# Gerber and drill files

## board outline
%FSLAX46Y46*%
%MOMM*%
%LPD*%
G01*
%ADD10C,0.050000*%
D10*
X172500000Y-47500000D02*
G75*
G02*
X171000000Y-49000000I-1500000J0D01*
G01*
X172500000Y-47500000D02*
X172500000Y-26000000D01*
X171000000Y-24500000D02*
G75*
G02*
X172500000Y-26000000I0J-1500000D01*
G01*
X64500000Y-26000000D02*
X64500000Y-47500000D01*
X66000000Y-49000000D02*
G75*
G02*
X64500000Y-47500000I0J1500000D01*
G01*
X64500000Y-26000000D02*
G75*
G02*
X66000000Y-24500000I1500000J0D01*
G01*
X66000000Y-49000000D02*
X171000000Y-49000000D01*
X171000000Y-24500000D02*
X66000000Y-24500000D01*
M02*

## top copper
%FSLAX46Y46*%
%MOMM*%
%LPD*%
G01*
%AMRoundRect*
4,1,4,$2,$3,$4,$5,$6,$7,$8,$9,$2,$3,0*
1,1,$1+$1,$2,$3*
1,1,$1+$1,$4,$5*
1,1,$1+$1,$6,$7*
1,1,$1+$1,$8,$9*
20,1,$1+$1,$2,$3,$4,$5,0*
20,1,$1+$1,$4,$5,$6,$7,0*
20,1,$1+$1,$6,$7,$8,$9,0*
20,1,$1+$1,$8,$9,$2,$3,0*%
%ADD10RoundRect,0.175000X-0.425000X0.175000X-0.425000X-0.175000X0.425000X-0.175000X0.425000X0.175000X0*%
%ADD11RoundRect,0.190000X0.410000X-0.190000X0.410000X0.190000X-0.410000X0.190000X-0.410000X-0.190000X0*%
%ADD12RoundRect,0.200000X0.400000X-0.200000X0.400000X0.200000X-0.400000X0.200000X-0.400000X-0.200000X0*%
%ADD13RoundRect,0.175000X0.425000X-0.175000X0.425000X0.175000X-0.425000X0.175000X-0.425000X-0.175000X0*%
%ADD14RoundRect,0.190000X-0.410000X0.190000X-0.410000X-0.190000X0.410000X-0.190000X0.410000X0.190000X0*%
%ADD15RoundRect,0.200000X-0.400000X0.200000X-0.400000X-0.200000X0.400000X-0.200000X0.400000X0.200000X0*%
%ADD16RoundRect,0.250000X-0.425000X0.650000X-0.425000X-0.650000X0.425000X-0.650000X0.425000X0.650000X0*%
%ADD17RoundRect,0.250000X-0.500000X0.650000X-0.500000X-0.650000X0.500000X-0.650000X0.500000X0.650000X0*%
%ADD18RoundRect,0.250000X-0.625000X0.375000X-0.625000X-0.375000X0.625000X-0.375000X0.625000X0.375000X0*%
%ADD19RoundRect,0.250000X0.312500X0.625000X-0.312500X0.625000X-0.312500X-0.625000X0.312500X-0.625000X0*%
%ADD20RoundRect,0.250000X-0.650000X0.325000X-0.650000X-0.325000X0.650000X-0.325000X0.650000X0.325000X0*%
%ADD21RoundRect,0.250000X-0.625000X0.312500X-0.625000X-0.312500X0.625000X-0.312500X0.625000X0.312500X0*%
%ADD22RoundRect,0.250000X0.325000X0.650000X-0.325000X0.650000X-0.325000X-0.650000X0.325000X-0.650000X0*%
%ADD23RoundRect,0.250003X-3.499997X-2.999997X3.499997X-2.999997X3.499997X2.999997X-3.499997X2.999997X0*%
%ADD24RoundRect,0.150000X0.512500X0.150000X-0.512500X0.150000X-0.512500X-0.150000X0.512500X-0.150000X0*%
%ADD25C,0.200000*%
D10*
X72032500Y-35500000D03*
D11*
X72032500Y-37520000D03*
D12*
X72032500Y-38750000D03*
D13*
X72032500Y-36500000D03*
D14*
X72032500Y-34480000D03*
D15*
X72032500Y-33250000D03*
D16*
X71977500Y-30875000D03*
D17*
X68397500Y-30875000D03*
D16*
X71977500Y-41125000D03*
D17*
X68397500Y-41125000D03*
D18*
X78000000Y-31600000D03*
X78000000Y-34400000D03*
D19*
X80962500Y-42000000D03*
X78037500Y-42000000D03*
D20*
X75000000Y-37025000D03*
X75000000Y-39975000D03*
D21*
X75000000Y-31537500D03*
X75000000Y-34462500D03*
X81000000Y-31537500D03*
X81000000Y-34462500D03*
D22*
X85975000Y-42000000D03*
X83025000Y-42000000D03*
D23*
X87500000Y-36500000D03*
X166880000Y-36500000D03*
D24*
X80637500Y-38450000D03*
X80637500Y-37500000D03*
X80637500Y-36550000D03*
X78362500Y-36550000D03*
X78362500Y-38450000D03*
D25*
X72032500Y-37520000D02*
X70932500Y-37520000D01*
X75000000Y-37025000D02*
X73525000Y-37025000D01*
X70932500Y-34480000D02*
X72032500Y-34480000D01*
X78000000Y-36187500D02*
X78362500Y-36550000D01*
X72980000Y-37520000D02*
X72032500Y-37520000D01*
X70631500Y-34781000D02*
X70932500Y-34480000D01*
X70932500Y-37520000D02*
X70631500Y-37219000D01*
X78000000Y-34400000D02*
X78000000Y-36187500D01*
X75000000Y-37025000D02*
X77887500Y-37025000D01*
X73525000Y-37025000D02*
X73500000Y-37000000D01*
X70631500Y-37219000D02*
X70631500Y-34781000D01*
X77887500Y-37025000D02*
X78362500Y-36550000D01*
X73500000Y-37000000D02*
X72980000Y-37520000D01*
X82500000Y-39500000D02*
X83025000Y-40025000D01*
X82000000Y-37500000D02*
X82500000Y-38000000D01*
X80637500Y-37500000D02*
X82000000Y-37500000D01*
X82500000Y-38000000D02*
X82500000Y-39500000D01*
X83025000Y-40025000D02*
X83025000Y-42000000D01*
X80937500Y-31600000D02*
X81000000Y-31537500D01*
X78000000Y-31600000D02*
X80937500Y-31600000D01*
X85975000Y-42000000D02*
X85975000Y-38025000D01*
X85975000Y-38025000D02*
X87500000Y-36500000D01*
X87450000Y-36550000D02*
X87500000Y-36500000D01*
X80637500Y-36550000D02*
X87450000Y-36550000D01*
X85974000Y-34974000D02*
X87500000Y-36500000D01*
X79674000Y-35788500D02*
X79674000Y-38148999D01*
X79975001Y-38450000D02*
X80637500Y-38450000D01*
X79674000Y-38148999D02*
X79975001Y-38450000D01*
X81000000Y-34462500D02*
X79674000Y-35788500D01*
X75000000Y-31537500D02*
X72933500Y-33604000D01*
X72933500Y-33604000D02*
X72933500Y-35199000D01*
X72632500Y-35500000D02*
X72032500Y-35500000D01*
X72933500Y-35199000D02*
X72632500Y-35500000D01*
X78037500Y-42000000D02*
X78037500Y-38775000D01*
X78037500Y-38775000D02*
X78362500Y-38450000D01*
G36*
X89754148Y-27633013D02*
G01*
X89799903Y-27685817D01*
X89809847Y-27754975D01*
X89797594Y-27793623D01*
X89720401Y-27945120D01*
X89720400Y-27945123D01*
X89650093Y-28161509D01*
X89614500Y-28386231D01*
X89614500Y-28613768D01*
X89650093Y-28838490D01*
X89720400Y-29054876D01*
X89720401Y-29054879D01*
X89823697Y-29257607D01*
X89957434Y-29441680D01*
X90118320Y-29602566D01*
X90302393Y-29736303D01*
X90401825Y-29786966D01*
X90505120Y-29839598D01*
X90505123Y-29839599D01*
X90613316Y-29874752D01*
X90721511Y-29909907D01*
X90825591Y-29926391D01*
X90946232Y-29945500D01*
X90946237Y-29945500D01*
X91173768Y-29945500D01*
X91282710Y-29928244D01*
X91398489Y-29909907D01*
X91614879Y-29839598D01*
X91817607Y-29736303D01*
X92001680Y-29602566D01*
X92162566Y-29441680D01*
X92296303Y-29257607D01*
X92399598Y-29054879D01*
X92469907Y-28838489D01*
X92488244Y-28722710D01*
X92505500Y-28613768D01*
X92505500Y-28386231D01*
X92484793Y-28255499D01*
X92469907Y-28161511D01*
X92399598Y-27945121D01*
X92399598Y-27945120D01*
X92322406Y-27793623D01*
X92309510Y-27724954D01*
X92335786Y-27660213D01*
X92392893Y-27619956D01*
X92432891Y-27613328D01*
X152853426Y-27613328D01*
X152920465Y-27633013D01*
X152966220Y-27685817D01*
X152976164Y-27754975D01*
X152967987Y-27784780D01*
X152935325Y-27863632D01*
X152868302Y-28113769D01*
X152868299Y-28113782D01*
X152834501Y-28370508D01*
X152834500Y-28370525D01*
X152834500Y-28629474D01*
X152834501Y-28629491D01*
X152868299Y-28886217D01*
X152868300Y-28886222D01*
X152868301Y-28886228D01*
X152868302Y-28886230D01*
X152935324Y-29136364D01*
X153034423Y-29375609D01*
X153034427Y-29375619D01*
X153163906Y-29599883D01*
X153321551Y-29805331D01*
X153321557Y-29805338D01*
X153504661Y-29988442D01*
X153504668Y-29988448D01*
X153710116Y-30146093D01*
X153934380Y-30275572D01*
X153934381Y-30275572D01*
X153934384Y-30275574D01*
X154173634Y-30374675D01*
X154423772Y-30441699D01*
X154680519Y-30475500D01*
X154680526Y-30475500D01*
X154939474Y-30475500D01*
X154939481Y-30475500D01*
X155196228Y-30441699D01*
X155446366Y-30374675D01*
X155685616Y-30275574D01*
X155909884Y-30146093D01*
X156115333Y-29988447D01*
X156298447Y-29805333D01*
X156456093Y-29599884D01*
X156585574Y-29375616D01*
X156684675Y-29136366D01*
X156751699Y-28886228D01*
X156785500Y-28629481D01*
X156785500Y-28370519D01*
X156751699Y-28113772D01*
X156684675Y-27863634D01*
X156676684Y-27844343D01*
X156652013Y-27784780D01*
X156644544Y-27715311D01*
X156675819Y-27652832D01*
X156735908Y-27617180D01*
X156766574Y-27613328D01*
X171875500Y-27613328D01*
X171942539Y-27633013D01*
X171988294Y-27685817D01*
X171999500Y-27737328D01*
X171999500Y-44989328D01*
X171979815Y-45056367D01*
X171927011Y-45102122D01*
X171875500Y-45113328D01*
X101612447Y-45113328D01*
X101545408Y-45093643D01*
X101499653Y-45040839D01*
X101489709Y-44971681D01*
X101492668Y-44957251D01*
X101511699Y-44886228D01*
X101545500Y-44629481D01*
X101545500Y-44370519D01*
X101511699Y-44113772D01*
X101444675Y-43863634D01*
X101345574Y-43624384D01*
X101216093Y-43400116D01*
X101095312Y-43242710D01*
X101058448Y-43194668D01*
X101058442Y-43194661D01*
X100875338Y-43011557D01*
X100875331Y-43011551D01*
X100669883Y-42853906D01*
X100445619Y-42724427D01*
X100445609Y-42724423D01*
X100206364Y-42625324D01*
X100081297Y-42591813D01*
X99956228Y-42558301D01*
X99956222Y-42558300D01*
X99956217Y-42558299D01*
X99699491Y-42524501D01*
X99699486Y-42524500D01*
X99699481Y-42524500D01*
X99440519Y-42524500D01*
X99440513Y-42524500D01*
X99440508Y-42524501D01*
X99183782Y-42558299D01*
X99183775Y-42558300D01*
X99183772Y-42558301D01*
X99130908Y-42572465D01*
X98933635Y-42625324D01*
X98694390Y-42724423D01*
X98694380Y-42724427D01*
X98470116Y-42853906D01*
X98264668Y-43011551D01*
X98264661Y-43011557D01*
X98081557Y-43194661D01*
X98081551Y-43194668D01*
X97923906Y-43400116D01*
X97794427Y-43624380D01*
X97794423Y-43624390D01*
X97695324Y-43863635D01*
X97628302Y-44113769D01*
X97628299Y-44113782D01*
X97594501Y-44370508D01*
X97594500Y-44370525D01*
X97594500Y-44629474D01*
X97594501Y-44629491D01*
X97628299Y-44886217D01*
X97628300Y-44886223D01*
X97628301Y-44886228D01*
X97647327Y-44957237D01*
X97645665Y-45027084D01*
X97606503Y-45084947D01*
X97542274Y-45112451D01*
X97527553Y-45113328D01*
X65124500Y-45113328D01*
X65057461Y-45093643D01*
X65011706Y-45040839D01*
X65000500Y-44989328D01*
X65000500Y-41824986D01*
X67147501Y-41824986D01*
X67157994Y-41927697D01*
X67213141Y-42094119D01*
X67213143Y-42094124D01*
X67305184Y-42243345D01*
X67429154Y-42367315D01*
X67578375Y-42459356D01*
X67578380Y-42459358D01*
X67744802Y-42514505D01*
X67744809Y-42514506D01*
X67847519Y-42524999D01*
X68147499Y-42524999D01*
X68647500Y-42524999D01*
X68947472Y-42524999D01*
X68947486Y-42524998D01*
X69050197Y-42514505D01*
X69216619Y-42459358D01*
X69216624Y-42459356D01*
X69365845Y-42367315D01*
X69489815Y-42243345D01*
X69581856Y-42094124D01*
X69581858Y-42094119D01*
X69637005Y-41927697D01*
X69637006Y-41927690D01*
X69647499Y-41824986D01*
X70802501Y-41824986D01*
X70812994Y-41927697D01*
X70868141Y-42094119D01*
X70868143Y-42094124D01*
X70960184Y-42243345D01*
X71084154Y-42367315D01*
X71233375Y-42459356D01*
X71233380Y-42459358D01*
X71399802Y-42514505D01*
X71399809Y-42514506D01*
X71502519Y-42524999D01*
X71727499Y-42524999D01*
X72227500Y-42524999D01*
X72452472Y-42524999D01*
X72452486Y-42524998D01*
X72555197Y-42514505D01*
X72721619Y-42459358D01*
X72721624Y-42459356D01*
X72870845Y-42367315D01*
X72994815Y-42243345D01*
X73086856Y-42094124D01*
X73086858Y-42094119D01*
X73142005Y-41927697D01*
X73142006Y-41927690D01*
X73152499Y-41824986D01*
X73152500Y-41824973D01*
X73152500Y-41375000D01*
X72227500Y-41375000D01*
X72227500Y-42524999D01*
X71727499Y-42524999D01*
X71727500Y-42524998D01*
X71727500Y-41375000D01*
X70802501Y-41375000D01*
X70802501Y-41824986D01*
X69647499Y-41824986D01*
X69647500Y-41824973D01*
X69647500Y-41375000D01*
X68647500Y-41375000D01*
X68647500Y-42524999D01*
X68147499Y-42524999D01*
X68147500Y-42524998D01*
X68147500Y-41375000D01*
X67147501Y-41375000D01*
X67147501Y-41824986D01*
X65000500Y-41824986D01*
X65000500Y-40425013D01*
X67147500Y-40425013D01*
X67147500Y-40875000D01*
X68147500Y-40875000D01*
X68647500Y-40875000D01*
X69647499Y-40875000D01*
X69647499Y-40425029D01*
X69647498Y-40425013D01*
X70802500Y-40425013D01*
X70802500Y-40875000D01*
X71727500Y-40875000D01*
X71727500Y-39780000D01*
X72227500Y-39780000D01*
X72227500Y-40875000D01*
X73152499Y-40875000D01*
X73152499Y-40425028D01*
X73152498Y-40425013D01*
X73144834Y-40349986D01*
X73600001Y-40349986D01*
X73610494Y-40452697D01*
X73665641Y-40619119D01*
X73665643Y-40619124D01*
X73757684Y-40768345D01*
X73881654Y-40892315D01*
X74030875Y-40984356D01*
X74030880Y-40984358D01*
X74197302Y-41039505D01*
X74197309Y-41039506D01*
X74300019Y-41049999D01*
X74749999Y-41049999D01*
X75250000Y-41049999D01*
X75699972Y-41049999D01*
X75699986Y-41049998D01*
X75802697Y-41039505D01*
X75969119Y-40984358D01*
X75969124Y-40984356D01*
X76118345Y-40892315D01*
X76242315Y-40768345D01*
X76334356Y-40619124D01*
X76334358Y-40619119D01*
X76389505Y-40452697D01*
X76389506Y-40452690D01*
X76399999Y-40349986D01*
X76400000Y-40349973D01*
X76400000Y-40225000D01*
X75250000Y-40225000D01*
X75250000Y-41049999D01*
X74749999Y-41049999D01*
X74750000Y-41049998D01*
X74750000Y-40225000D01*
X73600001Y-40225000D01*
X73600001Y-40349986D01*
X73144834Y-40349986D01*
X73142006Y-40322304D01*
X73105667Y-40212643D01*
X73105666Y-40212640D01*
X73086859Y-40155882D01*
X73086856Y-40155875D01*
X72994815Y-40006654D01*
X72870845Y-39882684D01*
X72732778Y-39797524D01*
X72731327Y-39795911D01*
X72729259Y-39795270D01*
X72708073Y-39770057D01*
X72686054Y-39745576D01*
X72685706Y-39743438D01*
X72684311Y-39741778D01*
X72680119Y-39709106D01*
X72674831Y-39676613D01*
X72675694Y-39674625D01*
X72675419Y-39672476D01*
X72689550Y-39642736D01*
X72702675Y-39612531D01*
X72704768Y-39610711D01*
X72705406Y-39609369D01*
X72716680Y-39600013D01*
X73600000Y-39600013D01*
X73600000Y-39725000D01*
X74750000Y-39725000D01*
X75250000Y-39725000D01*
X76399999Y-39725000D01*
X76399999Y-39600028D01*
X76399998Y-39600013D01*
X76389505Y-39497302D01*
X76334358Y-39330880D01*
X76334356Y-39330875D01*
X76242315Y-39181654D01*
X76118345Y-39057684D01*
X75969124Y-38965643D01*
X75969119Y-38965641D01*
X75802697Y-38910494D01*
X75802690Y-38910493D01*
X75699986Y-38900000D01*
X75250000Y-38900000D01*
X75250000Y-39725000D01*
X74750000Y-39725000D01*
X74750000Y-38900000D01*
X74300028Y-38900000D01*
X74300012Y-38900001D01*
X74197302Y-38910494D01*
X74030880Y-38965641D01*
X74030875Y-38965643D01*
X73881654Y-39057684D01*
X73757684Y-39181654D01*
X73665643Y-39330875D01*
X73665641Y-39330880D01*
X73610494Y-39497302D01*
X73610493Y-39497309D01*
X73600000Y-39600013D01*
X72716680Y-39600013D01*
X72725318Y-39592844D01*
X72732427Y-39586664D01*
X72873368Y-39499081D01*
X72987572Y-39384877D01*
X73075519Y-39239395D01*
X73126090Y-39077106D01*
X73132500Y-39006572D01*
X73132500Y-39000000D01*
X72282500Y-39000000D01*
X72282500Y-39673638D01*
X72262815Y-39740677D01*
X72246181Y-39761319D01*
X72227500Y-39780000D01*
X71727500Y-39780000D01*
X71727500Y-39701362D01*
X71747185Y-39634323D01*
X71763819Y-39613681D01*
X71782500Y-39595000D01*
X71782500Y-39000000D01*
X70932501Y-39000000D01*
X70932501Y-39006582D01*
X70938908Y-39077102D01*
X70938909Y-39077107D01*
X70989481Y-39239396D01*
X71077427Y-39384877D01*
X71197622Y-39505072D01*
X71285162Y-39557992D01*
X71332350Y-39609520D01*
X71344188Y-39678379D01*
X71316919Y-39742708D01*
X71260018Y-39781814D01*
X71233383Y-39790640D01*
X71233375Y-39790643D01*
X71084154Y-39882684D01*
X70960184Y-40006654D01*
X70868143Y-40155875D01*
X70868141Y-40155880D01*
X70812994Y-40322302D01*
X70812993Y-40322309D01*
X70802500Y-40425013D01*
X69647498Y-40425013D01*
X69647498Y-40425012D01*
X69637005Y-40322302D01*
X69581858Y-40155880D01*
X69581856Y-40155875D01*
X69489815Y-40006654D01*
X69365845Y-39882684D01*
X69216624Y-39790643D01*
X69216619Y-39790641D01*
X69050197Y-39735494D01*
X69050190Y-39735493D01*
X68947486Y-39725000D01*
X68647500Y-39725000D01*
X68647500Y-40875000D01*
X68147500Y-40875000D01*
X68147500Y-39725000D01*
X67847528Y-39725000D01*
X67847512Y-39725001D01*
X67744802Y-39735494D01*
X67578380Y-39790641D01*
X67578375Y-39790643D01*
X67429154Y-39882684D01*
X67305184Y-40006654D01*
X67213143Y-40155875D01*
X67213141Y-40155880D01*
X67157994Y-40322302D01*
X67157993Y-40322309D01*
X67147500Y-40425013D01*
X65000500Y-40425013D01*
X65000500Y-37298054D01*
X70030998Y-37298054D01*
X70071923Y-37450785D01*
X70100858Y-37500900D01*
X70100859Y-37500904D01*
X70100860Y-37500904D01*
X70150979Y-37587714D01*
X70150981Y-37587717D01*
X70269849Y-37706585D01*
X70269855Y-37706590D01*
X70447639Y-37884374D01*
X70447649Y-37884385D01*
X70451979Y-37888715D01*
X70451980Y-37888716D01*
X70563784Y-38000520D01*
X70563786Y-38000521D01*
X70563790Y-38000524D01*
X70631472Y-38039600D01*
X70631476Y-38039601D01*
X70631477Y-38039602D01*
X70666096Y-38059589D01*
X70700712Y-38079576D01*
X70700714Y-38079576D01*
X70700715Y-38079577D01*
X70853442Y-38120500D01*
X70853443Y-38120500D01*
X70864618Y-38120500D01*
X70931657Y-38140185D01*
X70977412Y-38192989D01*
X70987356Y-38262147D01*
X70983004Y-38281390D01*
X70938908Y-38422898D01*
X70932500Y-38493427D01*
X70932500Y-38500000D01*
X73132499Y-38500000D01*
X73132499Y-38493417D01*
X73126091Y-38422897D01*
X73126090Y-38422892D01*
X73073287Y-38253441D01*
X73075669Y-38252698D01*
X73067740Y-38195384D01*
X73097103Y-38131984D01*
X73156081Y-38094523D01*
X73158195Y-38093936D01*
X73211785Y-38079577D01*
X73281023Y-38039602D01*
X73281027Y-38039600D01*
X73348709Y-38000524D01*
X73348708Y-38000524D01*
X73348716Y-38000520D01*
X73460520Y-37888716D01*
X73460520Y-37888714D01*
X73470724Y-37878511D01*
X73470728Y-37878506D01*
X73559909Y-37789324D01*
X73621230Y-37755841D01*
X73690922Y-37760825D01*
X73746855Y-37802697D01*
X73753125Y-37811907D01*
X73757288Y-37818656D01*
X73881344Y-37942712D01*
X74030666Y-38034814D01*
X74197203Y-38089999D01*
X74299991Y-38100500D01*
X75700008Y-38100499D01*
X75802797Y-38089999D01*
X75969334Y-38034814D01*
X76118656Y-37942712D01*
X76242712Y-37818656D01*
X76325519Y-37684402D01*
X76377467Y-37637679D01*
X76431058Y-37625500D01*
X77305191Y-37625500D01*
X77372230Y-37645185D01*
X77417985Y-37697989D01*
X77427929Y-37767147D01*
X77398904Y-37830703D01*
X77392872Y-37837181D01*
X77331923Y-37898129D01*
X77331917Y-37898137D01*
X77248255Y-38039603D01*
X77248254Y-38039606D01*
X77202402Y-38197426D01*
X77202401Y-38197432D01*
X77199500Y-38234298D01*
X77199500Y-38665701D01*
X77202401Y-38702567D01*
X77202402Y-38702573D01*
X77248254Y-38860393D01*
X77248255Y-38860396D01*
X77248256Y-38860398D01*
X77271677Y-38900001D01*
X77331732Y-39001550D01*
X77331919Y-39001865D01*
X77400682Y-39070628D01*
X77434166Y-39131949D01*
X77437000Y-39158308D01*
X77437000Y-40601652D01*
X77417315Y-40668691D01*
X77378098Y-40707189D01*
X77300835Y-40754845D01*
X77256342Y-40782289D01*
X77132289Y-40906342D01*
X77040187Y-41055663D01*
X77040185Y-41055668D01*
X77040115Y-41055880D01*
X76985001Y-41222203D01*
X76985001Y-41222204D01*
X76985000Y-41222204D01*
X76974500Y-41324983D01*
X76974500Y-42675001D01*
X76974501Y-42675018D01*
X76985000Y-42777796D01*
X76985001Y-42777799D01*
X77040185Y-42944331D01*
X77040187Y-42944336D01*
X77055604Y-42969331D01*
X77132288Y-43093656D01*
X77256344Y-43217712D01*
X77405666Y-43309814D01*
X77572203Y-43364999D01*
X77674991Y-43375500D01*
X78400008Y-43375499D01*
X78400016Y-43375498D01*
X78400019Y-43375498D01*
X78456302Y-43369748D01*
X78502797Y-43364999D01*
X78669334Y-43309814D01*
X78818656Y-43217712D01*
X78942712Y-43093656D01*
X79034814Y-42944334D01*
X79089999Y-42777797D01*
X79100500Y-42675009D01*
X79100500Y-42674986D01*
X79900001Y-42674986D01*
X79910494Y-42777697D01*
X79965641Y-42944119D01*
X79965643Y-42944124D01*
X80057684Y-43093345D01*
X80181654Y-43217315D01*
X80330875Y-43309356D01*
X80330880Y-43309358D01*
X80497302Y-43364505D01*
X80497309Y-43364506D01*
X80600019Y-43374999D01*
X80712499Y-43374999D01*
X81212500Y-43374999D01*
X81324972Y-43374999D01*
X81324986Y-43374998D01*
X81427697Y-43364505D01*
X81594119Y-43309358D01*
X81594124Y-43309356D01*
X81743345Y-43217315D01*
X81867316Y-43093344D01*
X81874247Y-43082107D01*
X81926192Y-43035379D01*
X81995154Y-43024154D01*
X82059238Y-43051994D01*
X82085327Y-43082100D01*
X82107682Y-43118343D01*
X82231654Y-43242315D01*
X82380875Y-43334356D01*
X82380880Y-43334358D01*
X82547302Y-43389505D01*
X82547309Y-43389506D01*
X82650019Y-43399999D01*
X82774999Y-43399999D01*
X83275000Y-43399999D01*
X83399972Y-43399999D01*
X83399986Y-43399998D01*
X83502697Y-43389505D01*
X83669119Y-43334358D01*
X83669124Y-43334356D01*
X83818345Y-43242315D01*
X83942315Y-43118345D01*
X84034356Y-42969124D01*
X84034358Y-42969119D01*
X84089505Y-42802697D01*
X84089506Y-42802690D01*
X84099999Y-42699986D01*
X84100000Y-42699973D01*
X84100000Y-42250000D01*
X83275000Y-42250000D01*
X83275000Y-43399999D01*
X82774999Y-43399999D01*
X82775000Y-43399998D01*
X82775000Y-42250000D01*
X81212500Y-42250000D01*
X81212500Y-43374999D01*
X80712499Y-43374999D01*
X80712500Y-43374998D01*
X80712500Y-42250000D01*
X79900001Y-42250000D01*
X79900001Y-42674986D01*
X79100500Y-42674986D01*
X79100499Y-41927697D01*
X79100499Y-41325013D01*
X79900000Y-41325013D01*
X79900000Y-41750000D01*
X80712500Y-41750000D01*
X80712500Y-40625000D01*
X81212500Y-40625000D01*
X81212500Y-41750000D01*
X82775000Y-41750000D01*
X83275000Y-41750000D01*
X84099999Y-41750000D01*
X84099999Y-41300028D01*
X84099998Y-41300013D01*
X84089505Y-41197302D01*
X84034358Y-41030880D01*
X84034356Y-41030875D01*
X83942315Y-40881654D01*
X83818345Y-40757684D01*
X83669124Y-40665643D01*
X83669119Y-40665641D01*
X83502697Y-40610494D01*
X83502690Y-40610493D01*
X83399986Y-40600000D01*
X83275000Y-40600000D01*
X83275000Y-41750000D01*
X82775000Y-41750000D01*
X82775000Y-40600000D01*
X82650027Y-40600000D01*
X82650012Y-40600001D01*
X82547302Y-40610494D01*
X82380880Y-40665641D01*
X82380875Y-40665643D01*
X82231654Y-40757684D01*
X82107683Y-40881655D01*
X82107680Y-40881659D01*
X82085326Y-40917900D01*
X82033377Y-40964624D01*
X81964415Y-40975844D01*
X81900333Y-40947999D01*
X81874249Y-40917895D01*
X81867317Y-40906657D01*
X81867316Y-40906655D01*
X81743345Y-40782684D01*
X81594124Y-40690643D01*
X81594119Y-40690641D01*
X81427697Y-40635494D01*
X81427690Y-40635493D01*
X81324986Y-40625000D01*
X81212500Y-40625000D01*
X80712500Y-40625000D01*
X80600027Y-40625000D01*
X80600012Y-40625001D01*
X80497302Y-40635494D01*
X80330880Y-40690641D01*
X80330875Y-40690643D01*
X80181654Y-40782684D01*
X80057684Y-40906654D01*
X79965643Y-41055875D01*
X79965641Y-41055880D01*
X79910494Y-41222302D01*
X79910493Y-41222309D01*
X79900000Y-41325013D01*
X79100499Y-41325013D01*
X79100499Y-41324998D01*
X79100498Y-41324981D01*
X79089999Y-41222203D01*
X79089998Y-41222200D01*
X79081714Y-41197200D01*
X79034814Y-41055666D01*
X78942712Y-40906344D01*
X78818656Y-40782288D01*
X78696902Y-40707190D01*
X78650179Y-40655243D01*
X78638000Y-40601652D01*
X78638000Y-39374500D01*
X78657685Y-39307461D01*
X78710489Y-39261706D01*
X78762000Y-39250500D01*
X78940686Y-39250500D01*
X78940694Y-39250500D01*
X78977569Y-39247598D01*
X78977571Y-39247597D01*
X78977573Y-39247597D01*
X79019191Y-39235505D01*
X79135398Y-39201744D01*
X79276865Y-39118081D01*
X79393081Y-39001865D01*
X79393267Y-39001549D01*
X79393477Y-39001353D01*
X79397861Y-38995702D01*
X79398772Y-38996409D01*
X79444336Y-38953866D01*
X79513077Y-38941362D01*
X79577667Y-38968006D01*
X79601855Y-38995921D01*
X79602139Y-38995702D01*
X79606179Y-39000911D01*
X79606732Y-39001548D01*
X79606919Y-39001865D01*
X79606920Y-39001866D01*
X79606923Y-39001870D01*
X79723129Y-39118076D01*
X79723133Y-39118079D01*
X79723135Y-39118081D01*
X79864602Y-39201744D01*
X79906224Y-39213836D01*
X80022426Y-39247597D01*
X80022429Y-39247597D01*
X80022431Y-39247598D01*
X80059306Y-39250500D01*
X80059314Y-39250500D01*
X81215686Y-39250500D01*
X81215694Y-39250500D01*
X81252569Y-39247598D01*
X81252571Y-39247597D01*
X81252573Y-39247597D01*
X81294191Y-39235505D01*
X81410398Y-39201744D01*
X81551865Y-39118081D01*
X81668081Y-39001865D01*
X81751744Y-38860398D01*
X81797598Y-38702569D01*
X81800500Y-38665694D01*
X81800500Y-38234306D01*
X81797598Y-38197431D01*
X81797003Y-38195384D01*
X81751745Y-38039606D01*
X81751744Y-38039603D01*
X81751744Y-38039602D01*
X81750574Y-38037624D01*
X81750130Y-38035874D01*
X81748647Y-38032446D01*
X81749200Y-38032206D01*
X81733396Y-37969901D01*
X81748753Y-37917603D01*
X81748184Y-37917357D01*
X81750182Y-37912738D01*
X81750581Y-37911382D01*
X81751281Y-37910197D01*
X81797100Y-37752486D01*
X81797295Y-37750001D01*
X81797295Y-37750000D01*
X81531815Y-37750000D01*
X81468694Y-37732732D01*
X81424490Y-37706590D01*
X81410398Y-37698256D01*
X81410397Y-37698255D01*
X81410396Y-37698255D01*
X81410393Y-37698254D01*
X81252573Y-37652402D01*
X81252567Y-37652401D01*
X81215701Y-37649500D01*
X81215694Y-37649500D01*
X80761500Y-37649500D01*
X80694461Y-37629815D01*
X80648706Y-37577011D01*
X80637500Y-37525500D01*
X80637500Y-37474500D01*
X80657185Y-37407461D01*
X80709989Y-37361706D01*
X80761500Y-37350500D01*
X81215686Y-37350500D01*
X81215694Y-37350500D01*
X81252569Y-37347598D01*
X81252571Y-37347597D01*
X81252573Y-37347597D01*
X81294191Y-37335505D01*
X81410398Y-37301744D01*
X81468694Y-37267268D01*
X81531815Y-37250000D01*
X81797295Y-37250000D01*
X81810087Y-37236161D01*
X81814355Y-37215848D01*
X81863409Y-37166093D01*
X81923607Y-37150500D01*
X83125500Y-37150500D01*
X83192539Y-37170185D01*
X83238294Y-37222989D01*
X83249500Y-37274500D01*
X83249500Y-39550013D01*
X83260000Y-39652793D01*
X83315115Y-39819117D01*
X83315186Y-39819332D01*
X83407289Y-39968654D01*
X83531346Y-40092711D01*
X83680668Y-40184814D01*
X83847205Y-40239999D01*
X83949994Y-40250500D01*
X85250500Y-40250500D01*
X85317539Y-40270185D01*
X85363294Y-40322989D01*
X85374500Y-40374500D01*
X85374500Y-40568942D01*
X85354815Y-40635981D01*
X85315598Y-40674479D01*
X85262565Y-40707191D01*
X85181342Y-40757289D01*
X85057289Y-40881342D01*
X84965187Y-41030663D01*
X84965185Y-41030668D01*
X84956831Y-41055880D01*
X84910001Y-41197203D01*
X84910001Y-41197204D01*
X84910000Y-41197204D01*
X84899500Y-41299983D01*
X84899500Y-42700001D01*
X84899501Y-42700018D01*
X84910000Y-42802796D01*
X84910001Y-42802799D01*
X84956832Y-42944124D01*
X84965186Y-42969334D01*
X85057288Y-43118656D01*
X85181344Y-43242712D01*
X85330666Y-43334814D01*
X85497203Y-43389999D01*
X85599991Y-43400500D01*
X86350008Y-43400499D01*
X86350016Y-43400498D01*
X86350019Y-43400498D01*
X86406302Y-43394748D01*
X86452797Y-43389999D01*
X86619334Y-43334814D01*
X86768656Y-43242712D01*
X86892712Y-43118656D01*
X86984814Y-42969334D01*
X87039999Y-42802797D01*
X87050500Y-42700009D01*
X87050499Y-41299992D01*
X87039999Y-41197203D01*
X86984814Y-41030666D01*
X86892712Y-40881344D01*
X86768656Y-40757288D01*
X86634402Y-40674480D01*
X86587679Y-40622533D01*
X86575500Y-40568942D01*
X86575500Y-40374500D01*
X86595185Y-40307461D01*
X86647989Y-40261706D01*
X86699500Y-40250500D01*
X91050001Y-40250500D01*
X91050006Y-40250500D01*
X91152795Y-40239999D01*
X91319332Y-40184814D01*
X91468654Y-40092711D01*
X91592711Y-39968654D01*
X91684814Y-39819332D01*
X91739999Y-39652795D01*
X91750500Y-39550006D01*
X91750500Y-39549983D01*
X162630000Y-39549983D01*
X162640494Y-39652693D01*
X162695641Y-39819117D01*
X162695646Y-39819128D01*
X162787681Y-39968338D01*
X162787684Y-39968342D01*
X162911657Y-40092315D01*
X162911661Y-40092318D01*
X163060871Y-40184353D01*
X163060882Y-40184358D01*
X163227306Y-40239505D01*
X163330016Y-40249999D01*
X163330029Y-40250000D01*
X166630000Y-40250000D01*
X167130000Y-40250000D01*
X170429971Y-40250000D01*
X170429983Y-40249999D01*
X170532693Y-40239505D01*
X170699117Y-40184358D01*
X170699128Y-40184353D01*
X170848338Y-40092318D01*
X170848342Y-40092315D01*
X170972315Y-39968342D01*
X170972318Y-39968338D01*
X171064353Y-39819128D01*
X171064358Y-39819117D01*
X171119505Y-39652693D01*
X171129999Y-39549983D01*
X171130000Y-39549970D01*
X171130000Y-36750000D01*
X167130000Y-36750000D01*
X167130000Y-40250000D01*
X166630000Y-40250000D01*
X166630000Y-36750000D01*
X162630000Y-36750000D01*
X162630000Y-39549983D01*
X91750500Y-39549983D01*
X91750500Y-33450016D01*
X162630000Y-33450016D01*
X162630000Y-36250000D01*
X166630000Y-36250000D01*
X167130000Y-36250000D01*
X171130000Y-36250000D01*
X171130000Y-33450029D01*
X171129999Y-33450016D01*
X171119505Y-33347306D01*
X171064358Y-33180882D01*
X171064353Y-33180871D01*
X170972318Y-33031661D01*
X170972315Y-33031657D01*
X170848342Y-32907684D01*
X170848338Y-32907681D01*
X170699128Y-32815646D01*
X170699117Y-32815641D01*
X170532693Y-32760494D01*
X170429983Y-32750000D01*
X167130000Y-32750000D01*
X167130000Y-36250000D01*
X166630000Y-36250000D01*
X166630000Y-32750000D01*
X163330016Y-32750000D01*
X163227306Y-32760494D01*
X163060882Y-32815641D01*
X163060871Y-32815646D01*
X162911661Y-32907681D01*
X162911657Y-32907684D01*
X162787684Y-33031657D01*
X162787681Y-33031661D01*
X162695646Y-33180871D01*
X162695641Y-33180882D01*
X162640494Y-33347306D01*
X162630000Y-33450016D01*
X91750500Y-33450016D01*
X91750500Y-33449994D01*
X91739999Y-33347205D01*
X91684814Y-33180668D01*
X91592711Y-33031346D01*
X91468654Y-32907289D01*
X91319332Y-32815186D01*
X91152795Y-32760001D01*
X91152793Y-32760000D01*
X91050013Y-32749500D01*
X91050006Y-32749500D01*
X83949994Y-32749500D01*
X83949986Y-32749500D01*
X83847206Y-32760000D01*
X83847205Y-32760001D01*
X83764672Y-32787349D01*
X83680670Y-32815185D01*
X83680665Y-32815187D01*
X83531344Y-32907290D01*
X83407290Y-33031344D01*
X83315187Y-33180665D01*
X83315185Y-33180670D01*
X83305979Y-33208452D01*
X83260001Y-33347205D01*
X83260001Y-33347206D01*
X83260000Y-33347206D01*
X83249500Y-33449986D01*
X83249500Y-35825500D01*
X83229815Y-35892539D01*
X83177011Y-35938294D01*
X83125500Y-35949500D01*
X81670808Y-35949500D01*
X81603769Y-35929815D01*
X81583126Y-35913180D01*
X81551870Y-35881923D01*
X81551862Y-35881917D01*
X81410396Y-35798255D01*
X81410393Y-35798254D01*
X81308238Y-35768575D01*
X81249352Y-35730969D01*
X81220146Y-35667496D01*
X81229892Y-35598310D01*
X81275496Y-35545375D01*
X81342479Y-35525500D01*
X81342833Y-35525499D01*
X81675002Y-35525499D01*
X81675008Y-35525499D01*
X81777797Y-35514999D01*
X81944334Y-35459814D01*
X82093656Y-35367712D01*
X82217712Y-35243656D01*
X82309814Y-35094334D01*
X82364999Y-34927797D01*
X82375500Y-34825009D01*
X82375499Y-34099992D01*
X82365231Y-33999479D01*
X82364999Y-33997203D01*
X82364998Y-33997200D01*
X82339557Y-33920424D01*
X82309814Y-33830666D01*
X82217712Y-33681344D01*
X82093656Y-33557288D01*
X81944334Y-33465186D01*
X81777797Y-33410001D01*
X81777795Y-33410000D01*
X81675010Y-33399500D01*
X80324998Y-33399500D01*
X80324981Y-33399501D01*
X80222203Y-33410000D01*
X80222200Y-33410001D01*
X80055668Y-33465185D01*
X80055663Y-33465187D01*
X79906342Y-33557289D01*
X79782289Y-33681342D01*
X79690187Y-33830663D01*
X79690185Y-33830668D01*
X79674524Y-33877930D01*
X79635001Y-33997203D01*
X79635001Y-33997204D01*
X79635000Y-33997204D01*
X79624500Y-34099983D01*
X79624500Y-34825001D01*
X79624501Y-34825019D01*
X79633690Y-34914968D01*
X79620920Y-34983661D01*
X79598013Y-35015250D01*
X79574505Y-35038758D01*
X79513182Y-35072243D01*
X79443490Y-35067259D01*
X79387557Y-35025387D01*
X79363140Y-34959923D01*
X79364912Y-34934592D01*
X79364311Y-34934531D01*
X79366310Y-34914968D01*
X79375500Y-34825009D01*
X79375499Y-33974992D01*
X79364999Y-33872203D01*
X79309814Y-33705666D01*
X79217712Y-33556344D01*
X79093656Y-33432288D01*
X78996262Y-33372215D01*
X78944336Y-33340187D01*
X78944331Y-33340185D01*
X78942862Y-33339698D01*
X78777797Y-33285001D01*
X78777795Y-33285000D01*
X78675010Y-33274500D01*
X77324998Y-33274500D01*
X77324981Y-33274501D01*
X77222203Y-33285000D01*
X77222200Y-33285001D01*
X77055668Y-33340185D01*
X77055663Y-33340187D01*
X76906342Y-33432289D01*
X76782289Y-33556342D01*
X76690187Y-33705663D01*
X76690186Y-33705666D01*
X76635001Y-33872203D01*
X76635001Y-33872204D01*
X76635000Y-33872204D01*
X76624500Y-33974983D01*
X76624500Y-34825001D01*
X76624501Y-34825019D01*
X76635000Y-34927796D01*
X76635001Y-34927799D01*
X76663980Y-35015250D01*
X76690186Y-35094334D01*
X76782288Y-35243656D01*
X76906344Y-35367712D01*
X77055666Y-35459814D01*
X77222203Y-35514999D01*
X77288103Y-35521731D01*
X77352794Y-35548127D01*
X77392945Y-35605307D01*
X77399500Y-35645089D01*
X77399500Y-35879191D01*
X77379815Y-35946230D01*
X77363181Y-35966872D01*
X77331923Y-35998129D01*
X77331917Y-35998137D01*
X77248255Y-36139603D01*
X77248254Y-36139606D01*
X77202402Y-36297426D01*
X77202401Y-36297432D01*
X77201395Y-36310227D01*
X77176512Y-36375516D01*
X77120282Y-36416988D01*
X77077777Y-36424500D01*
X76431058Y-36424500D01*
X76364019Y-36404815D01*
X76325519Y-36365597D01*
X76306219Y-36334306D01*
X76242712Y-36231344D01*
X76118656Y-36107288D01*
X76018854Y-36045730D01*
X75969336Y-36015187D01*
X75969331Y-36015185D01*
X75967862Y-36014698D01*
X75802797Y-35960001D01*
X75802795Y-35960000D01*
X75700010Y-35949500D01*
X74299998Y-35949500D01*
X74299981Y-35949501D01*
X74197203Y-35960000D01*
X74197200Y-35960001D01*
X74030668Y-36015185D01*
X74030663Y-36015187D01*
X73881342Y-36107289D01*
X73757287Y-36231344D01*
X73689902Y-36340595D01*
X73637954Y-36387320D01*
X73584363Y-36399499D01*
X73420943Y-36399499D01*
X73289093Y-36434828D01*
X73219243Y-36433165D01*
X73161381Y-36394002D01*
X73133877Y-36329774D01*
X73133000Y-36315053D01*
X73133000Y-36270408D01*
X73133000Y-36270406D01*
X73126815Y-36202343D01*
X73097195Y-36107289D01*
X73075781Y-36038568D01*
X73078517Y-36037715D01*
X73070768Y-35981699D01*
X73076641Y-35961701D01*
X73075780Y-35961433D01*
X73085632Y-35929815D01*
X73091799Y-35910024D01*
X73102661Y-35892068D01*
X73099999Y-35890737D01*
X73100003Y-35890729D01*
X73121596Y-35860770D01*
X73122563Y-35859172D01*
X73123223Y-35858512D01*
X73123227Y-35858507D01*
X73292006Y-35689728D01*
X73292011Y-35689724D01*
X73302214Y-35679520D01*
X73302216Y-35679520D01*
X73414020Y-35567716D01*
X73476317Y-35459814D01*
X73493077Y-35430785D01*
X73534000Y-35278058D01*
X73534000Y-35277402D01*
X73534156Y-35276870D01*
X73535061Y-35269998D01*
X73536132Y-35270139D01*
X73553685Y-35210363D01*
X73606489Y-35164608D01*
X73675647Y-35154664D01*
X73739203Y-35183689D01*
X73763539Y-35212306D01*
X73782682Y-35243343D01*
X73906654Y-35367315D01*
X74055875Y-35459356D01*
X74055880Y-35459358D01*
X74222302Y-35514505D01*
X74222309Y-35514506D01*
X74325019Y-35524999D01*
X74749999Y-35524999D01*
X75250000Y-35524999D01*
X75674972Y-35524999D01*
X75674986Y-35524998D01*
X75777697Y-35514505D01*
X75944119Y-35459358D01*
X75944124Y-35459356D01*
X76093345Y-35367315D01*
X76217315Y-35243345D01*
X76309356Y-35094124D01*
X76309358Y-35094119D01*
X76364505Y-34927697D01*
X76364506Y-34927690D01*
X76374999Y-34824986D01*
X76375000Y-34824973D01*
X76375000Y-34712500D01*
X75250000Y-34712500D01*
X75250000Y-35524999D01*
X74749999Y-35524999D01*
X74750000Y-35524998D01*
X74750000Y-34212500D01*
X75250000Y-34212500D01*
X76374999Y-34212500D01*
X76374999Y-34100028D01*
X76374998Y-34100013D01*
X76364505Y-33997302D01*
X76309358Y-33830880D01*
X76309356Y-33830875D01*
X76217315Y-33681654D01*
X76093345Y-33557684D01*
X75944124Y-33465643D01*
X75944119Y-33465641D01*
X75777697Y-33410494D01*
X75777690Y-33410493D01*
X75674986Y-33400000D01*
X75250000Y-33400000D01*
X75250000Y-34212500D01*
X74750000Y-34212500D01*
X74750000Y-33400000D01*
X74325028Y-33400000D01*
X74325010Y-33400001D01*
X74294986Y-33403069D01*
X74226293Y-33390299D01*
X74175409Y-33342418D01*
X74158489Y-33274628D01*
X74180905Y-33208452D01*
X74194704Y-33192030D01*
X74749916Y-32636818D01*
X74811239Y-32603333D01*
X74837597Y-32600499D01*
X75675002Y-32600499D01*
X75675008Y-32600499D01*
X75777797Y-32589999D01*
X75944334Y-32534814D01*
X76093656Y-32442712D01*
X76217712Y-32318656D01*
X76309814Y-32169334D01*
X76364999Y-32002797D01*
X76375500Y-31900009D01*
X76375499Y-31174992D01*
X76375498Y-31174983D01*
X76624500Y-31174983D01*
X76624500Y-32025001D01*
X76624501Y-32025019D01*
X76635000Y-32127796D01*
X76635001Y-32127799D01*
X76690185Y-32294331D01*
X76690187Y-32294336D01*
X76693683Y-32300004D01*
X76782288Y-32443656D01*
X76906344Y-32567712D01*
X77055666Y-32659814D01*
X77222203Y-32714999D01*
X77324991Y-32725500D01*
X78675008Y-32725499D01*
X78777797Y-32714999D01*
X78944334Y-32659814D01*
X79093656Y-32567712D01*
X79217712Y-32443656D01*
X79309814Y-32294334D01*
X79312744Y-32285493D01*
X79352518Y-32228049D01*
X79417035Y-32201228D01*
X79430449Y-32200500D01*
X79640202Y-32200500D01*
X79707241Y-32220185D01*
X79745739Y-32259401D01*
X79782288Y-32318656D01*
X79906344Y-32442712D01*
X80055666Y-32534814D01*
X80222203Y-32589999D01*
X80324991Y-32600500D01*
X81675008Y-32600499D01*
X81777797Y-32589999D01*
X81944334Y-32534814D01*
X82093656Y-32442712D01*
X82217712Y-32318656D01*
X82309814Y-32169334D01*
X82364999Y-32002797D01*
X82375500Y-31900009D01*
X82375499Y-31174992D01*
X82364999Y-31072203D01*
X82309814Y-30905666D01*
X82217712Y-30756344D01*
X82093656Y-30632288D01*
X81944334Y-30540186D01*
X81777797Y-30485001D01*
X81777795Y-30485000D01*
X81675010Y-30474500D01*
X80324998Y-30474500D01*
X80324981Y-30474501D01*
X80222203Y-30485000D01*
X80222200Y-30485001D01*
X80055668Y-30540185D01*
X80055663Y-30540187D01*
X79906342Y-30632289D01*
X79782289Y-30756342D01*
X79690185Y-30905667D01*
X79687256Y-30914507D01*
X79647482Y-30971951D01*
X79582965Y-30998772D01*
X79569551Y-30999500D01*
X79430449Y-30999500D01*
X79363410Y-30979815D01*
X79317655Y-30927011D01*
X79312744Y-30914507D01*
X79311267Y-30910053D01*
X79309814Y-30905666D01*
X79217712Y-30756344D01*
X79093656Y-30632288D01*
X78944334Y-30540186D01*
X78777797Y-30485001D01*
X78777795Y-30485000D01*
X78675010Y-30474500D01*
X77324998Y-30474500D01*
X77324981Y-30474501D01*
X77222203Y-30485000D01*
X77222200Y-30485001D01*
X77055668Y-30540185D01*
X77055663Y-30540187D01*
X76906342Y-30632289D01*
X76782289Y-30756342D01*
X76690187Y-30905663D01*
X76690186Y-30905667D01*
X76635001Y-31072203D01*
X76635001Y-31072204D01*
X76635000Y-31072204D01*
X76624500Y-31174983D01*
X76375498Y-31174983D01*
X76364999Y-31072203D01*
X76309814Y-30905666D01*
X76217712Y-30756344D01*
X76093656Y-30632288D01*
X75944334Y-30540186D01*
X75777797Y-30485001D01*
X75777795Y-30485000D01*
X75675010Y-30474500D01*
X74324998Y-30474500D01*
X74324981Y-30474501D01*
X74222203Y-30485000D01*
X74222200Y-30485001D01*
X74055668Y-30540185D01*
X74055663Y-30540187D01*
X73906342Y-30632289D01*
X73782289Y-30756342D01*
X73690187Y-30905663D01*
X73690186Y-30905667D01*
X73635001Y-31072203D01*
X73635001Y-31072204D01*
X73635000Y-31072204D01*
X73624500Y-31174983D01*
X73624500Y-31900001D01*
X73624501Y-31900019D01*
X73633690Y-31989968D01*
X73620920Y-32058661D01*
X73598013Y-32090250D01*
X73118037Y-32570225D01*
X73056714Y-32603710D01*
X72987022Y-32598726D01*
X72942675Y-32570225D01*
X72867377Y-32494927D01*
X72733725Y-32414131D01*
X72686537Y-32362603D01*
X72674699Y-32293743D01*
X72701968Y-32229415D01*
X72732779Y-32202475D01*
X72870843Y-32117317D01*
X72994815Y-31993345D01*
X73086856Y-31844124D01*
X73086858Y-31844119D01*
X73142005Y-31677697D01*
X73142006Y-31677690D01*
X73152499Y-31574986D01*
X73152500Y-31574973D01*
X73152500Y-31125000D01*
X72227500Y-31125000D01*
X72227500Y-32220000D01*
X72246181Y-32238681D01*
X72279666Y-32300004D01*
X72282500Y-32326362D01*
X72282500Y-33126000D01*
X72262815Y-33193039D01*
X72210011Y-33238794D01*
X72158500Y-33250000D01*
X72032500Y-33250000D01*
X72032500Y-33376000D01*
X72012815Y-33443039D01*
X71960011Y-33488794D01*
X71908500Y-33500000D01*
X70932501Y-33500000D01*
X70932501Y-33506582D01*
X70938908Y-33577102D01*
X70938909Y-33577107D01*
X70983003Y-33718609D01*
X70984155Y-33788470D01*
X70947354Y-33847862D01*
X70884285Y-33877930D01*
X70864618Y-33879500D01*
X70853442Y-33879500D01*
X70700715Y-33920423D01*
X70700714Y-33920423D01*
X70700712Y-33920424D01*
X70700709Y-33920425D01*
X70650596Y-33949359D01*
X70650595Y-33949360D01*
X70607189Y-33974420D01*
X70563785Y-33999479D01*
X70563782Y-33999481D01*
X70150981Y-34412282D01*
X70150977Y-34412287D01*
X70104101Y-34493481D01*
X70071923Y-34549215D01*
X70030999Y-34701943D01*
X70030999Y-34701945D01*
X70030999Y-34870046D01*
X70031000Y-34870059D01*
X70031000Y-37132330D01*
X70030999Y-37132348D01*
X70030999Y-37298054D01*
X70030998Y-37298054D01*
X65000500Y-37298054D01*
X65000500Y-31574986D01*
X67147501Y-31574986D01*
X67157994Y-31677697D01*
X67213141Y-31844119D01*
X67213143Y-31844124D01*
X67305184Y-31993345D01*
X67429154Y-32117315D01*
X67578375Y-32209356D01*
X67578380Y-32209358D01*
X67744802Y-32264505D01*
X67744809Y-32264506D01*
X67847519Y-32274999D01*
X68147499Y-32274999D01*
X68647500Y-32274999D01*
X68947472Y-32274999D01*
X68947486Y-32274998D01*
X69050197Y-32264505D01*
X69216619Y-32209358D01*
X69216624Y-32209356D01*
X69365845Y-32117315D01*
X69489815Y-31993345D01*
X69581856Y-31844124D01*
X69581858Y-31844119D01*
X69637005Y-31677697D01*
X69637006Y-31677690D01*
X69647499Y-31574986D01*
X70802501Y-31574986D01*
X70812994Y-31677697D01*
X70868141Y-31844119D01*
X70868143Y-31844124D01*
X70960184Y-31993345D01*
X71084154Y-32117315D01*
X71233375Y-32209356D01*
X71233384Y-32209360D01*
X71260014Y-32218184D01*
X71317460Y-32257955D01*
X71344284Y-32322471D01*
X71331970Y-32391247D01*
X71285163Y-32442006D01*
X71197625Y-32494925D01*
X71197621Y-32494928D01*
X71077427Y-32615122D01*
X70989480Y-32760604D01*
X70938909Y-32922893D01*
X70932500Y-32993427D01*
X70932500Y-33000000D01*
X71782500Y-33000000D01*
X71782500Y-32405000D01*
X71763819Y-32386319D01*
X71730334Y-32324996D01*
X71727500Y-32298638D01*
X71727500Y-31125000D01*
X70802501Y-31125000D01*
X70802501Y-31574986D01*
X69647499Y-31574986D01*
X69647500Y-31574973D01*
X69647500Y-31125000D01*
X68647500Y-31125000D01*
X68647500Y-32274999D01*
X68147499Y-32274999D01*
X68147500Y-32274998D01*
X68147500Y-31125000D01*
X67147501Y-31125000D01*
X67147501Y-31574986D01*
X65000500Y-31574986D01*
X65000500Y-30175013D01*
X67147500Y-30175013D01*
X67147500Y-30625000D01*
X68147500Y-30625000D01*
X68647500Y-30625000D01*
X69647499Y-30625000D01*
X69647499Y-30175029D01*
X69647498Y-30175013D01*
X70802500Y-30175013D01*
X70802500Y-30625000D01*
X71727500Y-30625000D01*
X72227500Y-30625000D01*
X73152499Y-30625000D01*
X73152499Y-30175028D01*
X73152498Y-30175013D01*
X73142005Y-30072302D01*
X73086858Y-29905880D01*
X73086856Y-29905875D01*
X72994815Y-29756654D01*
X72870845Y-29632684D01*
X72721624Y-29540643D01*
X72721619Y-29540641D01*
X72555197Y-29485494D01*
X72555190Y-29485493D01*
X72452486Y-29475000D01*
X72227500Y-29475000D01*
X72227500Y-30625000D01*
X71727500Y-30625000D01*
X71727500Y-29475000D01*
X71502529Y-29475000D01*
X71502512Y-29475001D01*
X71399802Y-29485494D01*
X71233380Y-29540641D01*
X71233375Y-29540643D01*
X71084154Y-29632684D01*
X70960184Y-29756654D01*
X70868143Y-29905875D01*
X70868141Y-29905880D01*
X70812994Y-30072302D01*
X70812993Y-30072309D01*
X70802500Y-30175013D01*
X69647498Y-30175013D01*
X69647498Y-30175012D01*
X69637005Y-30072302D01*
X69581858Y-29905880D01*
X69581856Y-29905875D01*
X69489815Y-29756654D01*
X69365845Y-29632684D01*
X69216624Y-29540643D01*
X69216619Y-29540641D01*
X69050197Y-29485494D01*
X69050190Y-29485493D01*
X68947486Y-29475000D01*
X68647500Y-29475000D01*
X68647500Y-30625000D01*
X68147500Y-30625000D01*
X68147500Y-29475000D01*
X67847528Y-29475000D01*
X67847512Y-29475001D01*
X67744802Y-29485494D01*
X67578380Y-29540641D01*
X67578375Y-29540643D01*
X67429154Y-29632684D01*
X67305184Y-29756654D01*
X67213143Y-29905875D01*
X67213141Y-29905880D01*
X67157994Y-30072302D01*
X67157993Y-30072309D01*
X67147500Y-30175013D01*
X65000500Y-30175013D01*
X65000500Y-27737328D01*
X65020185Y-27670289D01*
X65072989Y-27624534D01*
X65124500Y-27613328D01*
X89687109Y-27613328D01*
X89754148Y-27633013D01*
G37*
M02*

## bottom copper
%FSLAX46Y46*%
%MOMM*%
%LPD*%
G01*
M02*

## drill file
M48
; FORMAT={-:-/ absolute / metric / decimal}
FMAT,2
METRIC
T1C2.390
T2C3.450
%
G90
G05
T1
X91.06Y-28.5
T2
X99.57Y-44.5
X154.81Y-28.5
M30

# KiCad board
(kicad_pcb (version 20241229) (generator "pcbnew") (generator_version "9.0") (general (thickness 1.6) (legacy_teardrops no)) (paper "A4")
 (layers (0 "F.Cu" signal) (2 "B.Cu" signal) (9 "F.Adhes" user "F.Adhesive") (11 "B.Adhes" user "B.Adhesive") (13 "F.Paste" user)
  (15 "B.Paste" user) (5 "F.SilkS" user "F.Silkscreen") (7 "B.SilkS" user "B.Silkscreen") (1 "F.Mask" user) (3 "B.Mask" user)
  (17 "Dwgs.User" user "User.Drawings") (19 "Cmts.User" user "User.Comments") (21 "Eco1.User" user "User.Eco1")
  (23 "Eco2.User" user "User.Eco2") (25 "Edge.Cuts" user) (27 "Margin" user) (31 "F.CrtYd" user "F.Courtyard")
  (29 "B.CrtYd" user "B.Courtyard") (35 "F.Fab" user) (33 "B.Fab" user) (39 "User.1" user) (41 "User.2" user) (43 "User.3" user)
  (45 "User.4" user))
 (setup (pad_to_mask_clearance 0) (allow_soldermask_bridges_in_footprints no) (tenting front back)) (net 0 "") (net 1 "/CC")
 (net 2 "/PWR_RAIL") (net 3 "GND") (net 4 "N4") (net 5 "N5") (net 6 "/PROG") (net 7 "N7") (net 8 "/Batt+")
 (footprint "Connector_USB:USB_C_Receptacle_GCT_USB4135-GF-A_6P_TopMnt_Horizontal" (layer "F.Cu") (at 69 36 -90)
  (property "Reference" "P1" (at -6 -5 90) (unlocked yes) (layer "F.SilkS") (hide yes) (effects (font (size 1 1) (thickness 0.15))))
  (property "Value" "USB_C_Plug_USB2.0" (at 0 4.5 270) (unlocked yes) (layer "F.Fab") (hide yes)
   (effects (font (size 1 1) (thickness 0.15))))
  (pad "A5" smd roundrect (at -0.5 -3.0325 270) (size 0.7 1.2) (layers "F.Cu" "F.Mask" "F.Paste") (roundrect_rratio 0.25) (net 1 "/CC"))
  (pad "A9" smd roundrect (at 1.52 -3.0325 90) (size 0.76 1.2) (layers "F.Cu" "F.Mask" "F.Paste") (roundrect_rratio 0.25)
   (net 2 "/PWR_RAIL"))
  (pad "A12" smd roundrect (at 2.75 -3.0325 90) (size 0.8 1.2) (layers "F.Cu" "F.Mask" "F.Paste") (roundrect_rratio 0.25) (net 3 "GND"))
  (pad "B5" smd roundrect (at 0.5 -3.0325 90) (size 0.7 1.2) (layers "F.Cu" "F.Mask" "F.Paste") (roundrect_rratio 0.25) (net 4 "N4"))
  (pad "B9" smd roundrect (at -1.52 -3.0325 270) (size 0.76 1.2) (layers "F.Cu" "F.Mask" "F.Paste") (roundrect_rratio 0.25)
   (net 2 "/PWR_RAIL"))
  (pad "B12" smd roundrect (at -2.75 -3.0325 270) (size 0.8 1.2) (layers "F.Cu" "F.Mask" "F.Paste") (roundrect_rratio 0.25) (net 3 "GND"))
  (pad "S1" smd roundrect (at -5.125 -2.9775 270) (size 1.8 1.35) (layers "F.Cu" "F.Mask" "F.Paste") (roundrect_rratio 0.1851851852)
   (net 3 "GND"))
  (pad "S1" smd roundrect (at -5.125 0.6025 270) (size 1.8 1.5) (layers "F.Cu" "F.Mask" "F.Paste") (roundrect_rratio 0.1666666667)
   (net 3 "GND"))
  (pad "S1" smd roundrect (at 5.125 -2.9775 270) (size 1.8 1.35) (layers "F.Cu" "F.Mask" "F.Paste") (roundrect_rratio 0.1851851852)
   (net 3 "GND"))
  (pad "S1" smd roundrect (at 5.125 0.6025 270) (size 1.8 1.5) (layers "F.Cu" "F.Mask" "F.Paste") (roundrect_rratio 0.1666666667)
   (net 3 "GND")))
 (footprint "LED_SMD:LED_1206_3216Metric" (layer "F.Cu") (at 78 33 -90)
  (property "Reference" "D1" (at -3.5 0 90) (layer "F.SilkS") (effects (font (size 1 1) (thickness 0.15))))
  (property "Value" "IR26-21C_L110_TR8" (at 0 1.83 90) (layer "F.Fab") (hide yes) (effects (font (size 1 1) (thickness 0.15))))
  (pad "1" smd roundrect (at -1.4 0 270) (size 1.25 1.75) (layers "F.Cu" "F.Mask" "F.Paste") (roundrect_rratio 0.2) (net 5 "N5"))
  (pad "2" smd roundrect (at 1.4 0 270) (size 1.25 1.75) (layers "F.Cu" "F.Mask" "F.Paste") (roundrect_rratio 0.2) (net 2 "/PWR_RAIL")))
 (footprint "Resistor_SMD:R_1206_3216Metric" (layer "F.Cu") (at 79.5 42 180)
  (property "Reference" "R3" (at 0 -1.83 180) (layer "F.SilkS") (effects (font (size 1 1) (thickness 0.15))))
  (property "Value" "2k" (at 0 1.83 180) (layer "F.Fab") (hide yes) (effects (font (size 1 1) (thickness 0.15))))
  (pad "1" smd roundrect (at -1.4625 0 180) (size 1.125 1.75) (layers "F.Cu" "F.Mask" "F.Paste") (roundrect_rratio 0.222222) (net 3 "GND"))
  (pad "2" smd roundrect (at 1.4625 0 180) (size 1.125 1.75) (layers "F.Cu" "F.Mask" "F.Paste") (roundrect_rratio 0.222222) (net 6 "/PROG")))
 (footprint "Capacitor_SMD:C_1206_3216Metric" (layer "F.Cu") (at 75 38.5 -90)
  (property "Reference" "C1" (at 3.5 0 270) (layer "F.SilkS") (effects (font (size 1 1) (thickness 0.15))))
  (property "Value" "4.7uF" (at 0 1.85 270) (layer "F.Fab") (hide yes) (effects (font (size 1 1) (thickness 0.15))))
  (pad "1" smd roundrect (at -1.475 0 270) (size 1.15 1.8) (layers "F.Cu" "F.Mask" "F.Paste") (roundrect_rratio 0.217391)
   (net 2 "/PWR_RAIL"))
  (pad "2" smd roundrect (at 1.475 0 270) (size 1.15 1.8) (layers "F.Cu" "F.Mask" "F.Paste") (roundrect_rratio 0.217391) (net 3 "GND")))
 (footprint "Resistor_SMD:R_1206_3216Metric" (layer "F.Cu") (at 75 33 -90)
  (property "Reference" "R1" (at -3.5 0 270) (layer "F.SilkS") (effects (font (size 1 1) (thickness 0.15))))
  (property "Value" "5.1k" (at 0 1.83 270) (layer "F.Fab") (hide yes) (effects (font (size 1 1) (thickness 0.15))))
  (pad "1" smd roundrect (at -1.4625 0 270) (size 1.125 1.75) (layers "F.Cu" "F.Mask" "F.Paste") (roundrect_rratio 0.222222) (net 1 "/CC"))
  (pad "2" smd roundrect (at 1.4625 0 270) (size 1.125 1.75) (layers "F.Cu" "F.Mask" "F.Paste") (roundrect_rratio 0.222222) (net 3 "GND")))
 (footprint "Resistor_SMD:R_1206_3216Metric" (layer "F.Cu") (at 81 33 -90)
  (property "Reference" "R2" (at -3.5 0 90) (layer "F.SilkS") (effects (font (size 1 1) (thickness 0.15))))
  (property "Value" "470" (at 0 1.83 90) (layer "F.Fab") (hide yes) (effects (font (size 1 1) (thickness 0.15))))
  (pad "1" smd roundrect (at -1.4625 0 270) (size 1.125 1.75) (layers "F.Cu" "F.Mask" "F.Paste") (roundrect_rratio 0.222222) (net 5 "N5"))
  (pad "2" smd roundrect (at 1.4625 0 270) (size 1.125 1.75) (layers "F.Cu" "F.Mask" "F.Paste") (roundrect_rratio 0.222222) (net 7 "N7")))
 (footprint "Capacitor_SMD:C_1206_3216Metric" (layer "F.Cu") (at 84.5 42 180)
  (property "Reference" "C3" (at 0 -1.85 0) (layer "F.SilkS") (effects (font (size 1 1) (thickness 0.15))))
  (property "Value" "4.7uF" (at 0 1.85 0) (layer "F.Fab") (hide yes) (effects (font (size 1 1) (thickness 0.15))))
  (pad "1" smd roundrect (at -1.475 0 180) (size 1.15 1.8) (layers "F.Cu" "F.Mask" "F.Paste") (roundrect_rratio 0.217391) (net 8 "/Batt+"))
  (pad "2" smd roundrect (at 1.475 0 180) (size 1.15 1.8) (layers "F.Cu" "F.Mask" "F.Paste") (roundrect_rratio 0.217391) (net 3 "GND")))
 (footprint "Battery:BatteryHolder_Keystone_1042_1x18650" (layer "F.Cu") (at 127.19 36.5)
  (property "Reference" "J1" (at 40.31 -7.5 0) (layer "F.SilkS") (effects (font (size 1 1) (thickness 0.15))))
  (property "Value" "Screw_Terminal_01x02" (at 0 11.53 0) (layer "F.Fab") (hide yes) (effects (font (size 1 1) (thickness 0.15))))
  (pad "" np_thru_hole circle (at -36.13 -8) (size 2.39 2.39) (drill 2.39) (layers "*.Cu" "*.Mask"))
  (pad "" np_thru_hole circle (at -27.62 8) (size 3.45 3.45) (drill 3.45) (layers "*.Cu" "*.Mask"))
  (pad "" np_thru_hole circle (at 27.62 -8) (size 3.45 3.45) (drill 3.45) (layers "*.Cu" "*.Mask"))
  (pad "1" smd roundrect (at -39.69 0) (size 7.5 6.5) (layers "F.Cu" "F.Mask" "F.Paste") (roundrect_rratio 0.038462) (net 8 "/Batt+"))
  (pad "2" smd roundrect (at 39.69 0) (size 7.5 6.5) (layers "F.Cu" "F.Mask" "F.Paste") (roundrect_rratio 0.038462) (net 3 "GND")))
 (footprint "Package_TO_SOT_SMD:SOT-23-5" (layer "F.Cu") (at 79.5 37.5 180)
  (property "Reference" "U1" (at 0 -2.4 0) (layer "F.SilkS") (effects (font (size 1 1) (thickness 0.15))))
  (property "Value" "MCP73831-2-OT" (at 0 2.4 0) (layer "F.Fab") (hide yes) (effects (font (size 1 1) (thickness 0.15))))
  (pad "1" smd roundrect (at -1.1375 -0.95 180) (size 1.325 0.6) (layers "F.Cu" "F.Mask" "F.Paste") (roundrect_rratio 0.25) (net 7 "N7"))
  (pad "2" smd roundrect (at -1.1375 0 180) (size 1.325 0.6) (layers "F.Cu" "F.Mask" "F.Paste") (roundrect_rratio 0.25) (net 3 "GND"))
  (pad "3" smd roundrect (at -1.1375 0.95 180) (size 1.325 0.6) (layers "F.Cu" "F.Mask" "F.Paste") (roundrect_rratio 0.25) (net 8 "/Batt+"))
  (pad "4" smd roundrect (at 1.1375 0.95 180) (size 1.325 0.6) (layers "F.Cu" "F.Mask" "F.Paste") (roundrect_rratio 0.25)
   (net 2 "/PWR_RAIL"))
  (pad "5" smd roundrect (at 1.1375 -0.95 180) (size 1.325 0.6) (layers "F.Cu" "F.Mask" "F.Paste") (roundrect_rratio 0.25) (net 6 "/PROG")))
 (gr_arc (start 172.5 47.5) (mid 172.06066 48.56066) (end 171 49) (stroke (width 0.05) (type default)) (layer "Edge.Cuts"))
 (gr_line (start 172.5 47.5) (end 172.5 26) (stroke (width 0.05) (type default)) (layer "Edge.Cuts"))
 (gr_arc (start 171 24.5) (mid 172.06066 24.93934) (end 172.5 26) (stroke (width 0.05) (type default)) (layer "Edge.Cuts"))
 (gr_line (start 64.5 26) (end 64.5 47.5) (stroke (width 0.05) (type default)) (layer "Edge.Cuts"))
 (gr_arc (start 66 49) (mid 64.93934 48.56066) (end 64.5 47.5) (stroke (width 0.05) (type default)) (layer "Edge.Cuts"))
 (gr_arc (start 64.5 26) (mid 64.93934 24.93934) (end 66 24.5) (stroke (width 0.05) (type default)) (layer "Edge.Cuts"))
 (gr_line (start 66 49) (end 171 49) (stroke (width 0.05) (type default)) (layer "Edge.Cuts"))
 (gr_line (start 171 24.5) (end 66 24.5) (stroke (width 0.05) (type default)) (layer "Edge.Cuts"))
 (segment (start 72.0325 37.52) (end 70.9325 37.52) (width 0.2) (layer "F.Cu") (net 2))
 (segment (start 75 37.025) (end 73.525 37.025) (width 0.2) (layer "F.Cu") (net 2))
 (segment (start 70.9325 34.48) (end 72.0325 34.48) (width 0.2) (layer "F.Cu") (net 2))
 (segment (start 78 36.1875) (end 78.3625 36.55) (width 0.2) (layer "F.Cu") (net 2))
 (segment (start 72.98 37.52) (end 72.0325 37.52) (width 0.2) (layer "F.Cu") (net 2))
 (segment (start 70.6315 34.781) (end 70.9325 34.48) (width 0.2) (layer "F.Cu") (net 2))
 (segment (start 70.9325 37.52) (end 70.6315 37.219) (width 0.2) (layer "F.Cu") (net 2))
 (segment (start 78 34.4) (end 78 36.1875) (width 0.2) (layer "F.Cu") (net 2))
 (segment (start 75 37.025) (end 77.8875 37.025) (width 0.2) (layer "F.Cu") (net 2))
 (segment (start 73.525 37.025) (end 73.5 37) (width 0.2) (layer "F.Cu") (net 2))
 (segment (start 70.6315 37.219) (end 70.6315 34.781) (width 0.2) (layer "F.Cu") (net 2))
 (segment (start 77.8875 37.025) (end 78.3625 36.55) (width 0.2) (layer "F.Cu") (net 2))
 (segment (start 73.5 37) (end 72.98 37.52) (width 0.2) (layer "F.Cu") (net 2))
 (segment (start 82.5 39.5) (end 83.025 40.025) (width 0.2) (layer "F.Cu") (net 3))
 (segment (start 82 37.5) (end 82.5 38) (width 0.2) (layer "F.Cu") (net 3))
 (segment (start 80.6375 37.5) (end 82 37.5) (width 0.2) (layer "F.Cu") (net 3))
 (segment (start 82.5 38) (end 82.5 39.5) (width 0.2) (layer "F.Cu") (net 3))
 (segment (start 83.025 40.025) (end 83.025 42) (width 0.2) (layer "F.Cu") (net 3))
 (segment (start 80.9375 31.6) (end 81 31.5375) (width 0.2) (layer "F.Cu") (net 5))
 (segment (start 78 31.6) (end 80.9375 31.6) (width 0.2) (layer "F.Cu") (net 5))
 (segment (start 85.975 42) (end 85.975 38.025) (width 0.2) (layer "F.Cu") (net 8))
 (segment (start 85.975 38.025) (end 87.5 36.5) (width 0.2) (layer "F.Cu") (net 8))
 (segment (start 87.45 36.55) (end 87.5 36.5) (width 0.2) (layer "F.Cu") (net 8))
 (segment (start 80.6375 36.55) (end 87.45 36.55) (width 0.2) (layer "F.Cu") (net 8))
 (segment (start 85.974 34.974) (end 87.5 36.5) (width 0.2) (layer "F.Cu") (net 8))
 (segment (start 79.674 35.7885) (end 79.674 38.148999) (width 0.2) (layer "F.Cu") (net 7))
 (segment (start 79.975001 38.45) (end 80.6375 38.45) (width 0.2) (layer "F.Cu") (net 7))
 (segment (start 79.674 38.148999) (end 79.975001 38.45) (width 0.2) (layer "F.Cu") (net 7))
 (segment (start 81 34.4625) (end 79.674 35.7885) (width 0.2) (layer "F.Cu") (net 7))
 (segment (start 75 31.5375) (end 72.9335 33.604) (width 0.2) (layer "F.Cu") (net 1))
 (segment (start 72.9335 33.604) (end 72.9335 35.199) (width 0.2) (layer "F.Cu") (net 1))
 (segment (start 72.6325 35.5) (end 72.0325 35.5) (width 0.2) (layer "F.Cu") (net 1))
 (segment (start 72.9335 35.199) (end 72.6325 35.5) (width 0.2) (layer "F.Cu") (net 1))
 (segment (start 78.0375 42) (end 78.0375 38.775) (width 0.2) (layer "F.Cu") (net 6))
 (segment (start 78.0375 38.775) (end 78.3625 38.45) (width 0.2) (layer "F.Cu") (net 6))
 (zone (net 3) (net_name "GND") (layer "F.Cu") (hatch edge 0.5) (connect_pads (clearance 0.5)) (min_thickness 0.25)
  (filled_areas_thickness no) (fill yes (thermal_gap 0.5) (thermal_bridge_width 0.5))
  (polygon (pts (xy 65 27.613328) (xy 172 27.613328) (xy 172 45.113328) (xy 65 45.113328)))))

